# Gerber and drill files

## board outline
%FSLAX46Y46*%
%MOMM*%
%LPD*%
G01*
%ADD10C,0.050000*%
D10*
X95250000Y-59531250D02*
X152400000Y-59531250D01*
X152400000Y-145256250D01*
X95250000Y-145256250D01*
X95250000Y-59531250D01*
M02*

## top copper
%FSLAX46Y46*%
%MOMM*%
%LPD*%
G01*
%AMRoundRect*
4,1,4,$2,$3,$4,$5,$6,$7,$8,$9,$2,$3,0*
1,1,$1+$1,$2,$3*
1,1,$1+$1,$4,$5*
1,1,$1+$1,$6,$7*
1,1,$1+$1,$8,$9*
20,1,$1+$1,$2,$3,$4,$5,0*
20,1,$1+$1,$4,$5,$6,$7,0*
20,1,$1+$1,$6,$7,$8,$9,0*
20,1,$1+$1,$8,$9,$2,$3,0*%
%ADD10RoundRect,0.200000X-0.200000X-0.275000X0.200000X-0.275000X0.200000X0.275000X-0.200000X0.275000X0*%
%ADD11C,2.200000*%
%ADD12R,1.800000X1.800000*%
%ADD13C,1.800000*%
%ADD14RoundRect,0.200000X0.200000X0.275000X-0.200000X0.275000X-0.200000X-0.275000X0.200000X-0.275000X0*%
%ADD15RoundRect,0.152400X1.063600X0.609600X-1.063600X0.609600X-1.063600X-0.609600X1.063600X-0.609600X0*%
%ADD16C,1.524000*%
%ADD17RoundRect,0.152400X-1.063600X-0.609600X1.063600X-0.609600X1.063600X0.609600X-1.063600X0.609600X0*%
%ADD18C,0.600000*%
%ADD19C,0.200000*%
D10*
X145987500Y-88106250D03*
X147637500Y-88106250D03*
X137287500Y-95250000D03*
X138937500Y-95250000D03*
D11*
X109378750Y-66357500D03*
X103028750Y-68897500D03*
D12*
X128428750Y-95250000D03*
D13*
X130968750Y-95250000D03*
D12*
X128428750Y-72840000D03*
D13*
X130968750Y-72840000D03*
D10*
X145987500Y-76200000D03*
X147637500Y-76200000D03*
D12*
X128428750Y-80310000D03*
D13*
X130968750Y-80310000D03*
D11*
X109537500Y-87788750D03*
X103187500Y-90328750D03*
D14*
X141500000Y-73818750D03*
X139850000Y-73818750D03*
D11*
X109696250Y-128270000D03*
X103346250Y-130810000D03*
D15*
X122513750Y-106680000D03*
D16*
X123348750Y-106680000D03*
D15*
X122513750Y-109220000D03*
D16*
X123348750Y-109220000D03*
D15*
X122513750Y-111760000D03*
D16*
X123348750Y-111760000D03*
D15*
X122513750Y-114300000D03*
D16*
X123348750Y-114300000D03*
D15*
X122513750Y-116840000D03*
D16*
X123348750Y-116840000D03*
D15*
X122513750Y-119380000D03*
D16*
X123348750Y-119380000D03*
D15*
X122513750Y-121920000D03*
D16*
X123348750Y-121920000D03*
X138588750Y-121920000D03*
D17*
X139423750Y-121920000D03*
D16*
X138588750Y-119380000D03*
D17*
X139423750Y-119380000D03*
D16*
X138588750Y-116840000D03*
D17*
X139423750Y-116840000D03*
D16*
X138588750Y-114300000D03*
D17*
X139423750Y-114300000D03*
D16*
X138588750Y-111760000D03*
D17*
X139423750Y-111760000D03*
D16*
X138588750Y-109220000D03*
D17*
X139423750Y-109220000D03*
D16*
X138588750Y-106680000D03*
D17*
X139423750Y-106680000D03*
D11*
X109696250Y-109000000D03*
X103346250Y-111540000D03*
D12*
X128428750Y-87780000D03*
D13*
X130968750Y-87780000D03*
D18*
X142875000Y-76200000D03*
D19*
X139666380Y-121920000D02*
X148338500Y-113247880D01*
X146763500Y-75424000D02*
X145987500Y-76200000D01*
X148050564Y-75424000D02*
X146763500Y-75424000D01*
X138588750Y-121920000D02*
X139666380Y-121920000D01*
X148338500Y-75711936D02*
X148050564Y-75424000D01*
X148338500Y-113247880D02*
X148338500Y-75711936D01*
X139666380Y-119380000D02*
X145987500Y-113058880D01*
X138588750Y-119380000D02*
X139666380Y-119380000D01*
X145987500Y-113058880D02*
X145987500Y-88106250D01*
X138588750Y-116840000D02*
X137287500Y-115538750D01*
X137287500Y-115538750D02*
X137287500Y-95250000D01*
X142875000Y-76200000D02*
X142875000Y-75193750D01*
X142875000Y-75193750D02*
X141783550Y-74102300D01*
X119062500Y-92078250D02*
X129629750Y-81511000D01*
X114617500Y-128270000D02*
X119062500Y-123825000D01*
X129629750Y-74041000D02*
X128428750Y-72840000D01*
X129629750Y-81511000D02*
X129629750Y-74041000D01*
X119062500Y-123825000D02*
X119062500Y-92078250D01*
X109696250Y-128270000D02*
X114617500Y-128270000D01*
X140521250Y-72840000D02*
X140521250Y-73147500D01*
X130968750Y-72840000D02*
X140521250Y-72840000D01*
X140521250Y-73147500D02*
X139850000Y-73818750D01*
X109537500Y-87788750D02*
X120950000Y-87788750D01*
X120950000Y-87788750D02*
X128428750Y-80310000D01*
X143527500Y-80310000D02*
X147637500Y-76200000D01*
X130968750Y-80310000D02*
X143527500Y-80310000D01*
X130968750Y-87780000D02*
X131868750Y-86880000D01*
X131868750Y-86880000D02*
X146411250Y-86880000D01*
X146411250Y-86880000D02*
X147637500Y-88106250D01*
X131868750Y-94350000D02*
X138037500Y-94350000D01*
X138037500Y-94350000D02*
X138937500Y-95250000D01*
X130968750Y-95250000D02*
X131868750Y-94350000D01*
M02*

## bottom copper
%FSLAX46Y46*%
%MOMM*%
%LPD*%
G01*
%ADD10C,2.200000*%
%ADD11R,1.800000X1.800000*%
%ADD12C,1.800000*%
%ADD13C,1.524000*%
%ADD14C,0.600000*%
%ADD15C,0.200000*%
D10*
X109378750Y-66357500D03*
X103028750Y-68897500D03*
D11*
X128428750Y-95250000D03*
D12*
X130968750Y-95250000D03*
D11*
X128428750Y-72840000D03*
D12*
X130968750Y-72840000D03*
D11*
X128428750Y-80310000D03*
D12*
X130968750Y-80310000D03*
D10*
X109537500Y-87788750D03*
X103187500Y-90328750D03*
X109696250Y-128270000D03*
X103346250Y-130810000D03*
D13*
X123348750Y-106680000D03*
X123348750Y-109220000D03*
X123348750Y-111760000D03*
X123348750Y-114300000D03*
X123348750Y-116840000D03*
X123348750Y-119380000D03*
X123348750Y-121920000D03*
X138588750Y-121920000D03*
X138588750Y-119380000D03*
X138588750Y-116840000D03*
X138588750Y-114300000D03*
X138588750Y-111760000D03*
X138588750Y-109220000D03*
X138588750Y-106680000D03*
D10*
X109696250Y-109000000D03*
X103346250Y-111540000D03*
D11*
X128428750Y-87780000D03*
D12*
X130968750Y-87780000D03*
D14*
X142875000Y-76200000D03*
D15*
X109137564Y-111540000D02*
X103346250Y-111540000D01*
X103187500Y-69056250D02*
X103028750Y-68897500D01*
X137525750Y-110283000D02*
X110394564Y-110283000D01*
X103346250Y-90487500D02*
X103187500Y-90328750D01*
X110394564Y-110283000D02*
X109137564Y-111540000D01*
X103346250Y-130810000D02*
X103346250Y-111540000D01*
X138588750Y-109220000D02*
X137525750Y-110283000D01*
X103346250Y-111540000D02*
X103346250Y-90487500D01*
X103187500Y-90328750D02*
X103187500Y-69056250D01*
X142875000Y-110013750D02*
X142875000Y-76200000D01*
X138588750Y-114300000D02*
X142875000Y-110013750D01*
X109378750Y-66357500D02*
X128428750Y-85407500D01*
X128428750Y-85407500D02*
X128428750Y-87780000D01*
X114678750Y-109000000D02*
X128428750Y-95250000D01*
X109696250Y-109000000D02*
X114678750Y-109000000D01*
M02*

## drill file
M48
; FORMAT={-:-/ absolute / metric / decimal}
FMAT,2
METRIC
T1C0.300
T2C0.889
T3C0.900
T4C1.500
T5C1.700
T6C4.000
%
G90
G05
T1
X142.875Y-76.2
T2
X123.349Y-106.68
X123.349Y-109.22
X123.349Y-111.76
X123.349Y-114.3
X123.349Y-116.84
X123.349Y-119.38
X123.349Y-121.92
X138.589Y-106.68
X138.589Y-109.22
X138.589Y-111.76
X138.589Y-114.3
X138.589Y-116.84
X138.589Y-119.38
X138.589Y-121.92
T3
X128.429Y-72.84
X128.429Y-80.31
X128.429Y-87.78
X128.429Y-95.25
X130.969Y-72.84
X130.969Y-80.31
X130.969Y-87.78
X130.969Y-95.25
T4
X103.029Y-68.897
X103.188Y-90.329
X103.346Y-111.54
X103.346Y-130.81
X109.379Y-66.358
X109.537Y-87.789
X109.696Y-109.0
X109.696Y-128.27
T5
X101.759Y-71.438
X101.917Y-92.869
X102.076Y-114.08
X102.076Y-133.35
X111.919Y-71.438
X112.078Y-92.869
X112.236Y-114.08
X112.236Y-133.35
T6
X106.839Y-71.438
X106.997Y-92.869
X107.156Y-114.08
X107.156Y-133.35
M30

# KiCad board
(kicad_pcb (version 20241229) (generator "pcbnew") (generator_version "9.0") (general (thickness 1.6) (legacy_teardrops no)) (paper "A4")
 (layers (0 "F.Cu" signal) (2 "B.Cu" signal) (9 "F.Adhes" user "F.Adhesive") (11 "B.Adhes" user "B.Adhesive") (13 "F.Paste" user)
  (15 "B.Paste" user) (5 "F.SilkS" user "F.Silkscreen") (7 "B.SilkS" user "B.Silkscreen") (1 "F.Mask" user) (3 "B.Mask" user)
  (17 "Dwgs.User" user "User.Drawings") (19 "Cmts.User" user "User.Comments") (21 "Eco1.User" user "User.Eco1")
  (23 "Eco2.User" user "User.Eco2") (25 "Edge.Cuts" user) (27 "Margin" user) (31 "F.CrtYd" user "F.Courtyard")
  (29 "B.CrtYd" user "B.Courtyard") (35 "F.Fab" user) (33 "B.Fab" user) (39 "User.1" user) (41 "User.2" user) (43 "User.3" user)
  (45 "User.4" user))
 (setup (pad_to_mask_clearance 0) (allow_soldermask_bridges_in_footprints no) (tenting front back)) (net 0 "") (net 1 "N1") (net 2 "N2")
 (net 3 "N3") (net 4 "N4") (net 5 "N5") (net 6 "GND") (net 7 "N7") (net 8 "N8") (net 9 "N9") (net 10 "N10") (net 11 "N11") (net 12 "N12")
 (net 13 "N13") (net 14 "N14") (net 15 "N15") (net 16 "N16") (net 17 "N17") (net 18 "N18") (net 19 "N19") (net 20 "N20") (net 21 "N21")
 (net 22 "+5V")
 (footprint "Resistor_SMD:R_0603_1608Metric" (layer "F.Cu") (at 146.8125 88.10625)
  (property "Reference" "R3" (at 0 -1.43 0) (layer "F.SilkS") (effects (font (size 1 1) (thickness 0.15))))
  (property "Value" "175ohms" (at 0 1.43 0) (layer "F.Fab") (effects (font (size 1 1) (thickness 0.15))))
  (pad "1" smd roundrect (at -0.825 0) (size 0.8 0.95) (layers "F.Cu" "F.Mask" "F.Paste") (roundrect_rratio 0.25) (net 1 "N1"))
  (pad "2" smd roundrect (at 0.825 0) (size 0.8 0.95) (layers "F.Cu" "F.Mask" "F.Paste") (roundrect_rratio 0.25) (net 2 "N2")))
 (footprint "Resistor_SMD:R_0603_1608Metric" (layer "F.Cu") (at 138.1125 95.25)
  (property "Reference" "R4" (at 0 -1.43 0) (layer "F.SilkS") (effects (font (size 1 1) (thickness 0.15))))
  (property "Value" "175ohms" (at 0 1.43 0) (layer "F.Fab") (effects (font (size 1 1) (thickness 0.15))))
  (pad "1" smd roundrect (at -0.825 0) (size 0.8 0.95) (layers "F.Cu" "F.Mask" "F.Paste") (roundrect_rratio 0.25) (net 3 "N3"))
  (pad "2" smd roundrect (at 0.825 0) (size 0.8 0.95) (layers "F.Cu" "F.Mask" "F.Paste") (roundrect_rratio 0.25) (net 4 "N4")))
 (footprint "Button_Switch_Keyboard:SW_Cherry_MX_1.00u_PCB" (layer "F.Cu") (at 109.37875 66.3575)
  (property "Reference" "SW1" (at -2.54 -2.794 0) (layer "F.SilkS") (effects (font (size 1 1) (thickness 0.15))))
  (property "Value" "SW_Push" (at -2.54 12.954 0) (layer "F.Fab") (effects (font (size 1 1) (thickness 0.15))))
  (pad "" np_thru_hole circle (at -7.62 5.08) (size 1.7 1.7) (drill 1.7) (layers "*.Cu" "*.Mask"))
  (pad "" np_thru_hole circle (at -2.54 5.08) (size 4 4) (drill 4) (layers "*.Cu" "*.Mask"))
  (pad "" np_thru_hole circle (at 2.54 5.08) (size 1.7 1.7) (drill 1.7) (layers "*.Cu" "*.Mask"))
  (pad "1" thru_hole circle (at 0 0) (size 2.2 2.2) (drill 1.5) (layers "*.Cu" "*.Mask") (remove_unused_layers no) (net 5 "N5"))
  (pad "2" thru_hole circle (at -6.35 2.54) (size 2.2 2.2) (drill 1.5) (layers "*.Cu" "*.Mask") (remove_unused_layers no) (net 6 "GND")))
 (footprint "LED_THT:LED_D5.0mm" (layer "F.Cu") (at 128.42875 95.25)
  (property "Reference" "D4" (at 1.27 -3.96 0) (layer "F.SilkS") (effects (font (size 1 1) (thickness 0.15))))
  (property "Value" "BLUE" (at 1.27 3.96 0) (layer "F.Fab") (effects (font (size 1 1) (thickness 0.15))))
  (pad "1" thru_hole rect (at 0 0) (size 1.8 1.8) (drill 0.9) (layers "*.Cu" "*.Mask") (remove_unused_layers no) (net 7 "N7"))
  (pad "2" thru_hole circle (at 2.54 0) (size 1.8 1.8) (drill 0.9) (layers "*.Cu" "*.Mask") (remove_unused_layers no) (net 4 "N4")))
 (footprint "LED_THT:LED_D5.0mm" (layer "F.Cu") (at 128.42875 72.84)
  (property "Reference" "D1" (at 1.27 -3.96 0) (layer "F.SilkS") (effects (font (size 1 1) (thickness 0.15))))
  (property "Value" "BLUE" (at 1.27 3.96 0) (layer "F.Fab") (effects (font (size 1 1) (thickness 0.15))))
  (pad "1" thru_hole rect (at 0 0) (size 1.8 1.8) (drill 0.9) (layers "*.Cu" "*.Mask") (remove_unused_layers no) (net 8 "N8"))
  (pad "2" thru_hole circle (at 2.54 0) (size 1.8 1.8) (drill 0.9) (layers "*.Cu" "*.Mask") (remove_unused_layers no) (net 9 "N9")))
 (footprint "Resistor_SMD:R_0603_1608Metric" (layer "F.Cu") (at 146.8125 76.2)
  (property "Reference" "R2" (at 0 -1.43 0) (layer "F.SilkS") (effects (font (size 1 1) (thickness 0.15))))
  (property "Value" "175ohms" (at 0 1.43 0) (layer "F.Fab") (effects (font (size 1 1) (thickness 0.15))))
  (pad "1" smd roundrect (at -0.825 0) (size 0.8 0.95) (layers "F.Cu" "F.Mask" "F.Paste") (roundrect_rratio 0.25) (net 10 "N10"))
  (pad "2" smd roundrect (at 0.825 0) (size 0.8 0.95) (layers "F.Cu" "F.Mask" "F.Paste") (roundrect_rratio 0.25) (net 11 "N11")))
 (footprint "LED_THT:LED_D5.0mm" (layer "F.Cu") (at 128.42875 80.31)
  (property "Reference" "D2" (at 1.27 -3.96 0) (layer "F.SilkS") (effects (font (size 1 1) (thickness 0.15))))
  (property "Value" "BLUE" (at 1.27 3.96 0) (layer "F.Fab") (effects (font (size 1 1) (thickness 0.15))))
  (pad "1" thru_hole rect (at 0 0) (size 1.8 1.8) (drill 0.9) (layers "*.Cu" "*.Mask") (remove_unused_layers no) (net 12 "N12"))
  (pad "2" thru_hole circle (at 2.54 0) (size 1.8 1.8) (drill 0.9) (layers "*.Cu" "*.Mask") (remove_unused_layers no) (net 11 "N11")))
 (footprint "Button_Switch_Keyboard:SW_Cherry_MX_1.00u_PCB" (layer "F.Cu") (at 109.5375 87.78875)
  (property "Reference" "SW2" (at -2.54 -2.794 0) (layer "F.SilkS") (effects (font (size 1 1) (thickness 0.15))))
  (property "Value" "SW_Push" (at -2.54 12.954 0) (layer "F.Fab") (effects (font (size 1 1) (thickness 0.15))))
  (pad "" np_thru_hole circle (at -7.62 5.08) (size 1.7 1.7) (drill 1.7) (layers "*.Cu" "*.Mask"))
  (pad "" np_thru_hole circle (at -2.54 5.08) (size 4 4) (drill 4) (layers "*.Cu" "*.Mask"))
  (pad "" np_thru_hole circle (at 2.54 5.08) (size 1.7 1.7) (drill 1.7) (layers "*.Cu" "*.Mask"))
  (pad "1" thru_hole circle (at 0 0) (size 2.2 2.2) (drill 1.5) (layers "*.Cu" "*.Mask") (remove_unused_layers no) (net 12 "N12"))
  (pad "2" thru_hole circle (at -6.35 2.54) (size 2.2 2.2) (drill 1.5) (layers "*.Cu" "*.Mask") (remove_unused_layers no) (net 6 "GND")))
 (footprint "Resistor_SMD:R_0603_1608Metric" (layer "F.Cu") (at 140.675 73.81875 180)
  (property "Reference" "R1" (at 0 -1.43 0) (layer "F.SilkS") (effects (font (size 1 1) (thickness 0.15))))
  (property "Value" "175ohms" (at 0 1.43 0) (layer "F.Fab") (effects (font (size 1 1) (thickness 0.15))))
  (pad "1" smd roundrect (at -0.825 0 180) (size 0.8 0.95) (layers "F.Cu" "F.Mask" "F.Paste") (roundrect_rratio 0.25) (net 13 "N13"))
  (pad "2" smd roundrect (at 0.825 0 180) (size 0.8 0.95) (layers "F.Cu" "F.Mask" "F.Paste") (roundrect_rratio 0.25) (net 9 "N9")))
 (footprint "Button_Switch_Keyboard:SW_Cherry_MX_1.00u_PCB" (layer "F.Cu") (at 109.69625 128.27)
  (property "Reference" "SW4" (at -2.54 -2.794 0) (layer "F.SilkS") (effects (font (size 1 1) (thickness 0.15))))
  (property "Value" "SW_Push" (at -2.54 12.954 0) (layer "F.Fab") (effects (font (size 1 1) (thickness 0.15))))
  (pad "" np_thru_hole circle (at -7.62 5.08) (size 1.7 1.7) (drill 1.7) (layers "*.Cu" "*.Mask"))
  (pad "" np_thru_hole circle (at -2.54 5.08) (size 4 4) (drill 4) (layers "*.Cu" "*.Mask"))
  (pad "" np_thru_hole circle (at 2.54 5.08) (size 1.7 1.7) (drill 1.7) (layers "*.Cu" "*.Mask"))
  (pad "1" thru_hole circle (at 0 0) (size 2.2 2.2) (drill 1.5) (layers "*.Cu" "*.Mask") (remove_unused_layers no) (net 8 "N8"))
  (pad "2" thru_hole circle (at -6.35 2.54) (size 2.2 2.2) (drill 1.5) (layers "*.Cu" "*.Mask") (remove_unused_layers no) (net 6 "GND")))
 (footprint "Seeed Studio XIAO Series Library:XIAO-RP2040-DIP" (layer "F.Cu") (at 130.96875 114.3)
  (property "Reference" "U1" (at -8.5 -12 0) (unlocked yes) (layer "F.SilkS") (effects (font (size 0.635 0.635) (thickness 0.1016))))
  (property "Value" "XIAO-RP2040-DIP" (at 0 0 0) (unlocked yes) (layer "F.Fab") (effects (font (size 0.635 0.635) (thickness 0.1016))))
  (pad "1" smd roundrect (at -8.455 -7.62 180) (size 2.432 1.524) (layers "F.Cu" "F.Mask") (roundrect_rratio 0.1) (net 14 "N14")
   (thermal_bridge_angle 45))
  (pad "1" thru_hole circle (at -7.62 -7.62 180) (size 1.524 1.524) (drill 0.889) (layers "*.Cu" "*.Mask") (remove_unused_layers no)
   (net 14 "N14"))
  (pad "2" smd roundrect (at -8.455 -5.08 180) (size 2.432 1.524) (layers "F.Cu" "F.Mask") (roundrect_rratio 0.1) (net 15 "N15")
   (thermal_bridge_angle 45))
  (pad "2" thru_hole circle (at -7.62 -5.08 180) (size 1.524 1.524) (drill 0.889) (layers "*.Cu" "*.Mask") (remove_unused_layers no)
   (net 15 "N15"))
  (pad "3" smd roundrect (at -8.455 -2.54 180) (size 2.432 1.524) (layers "F.Cu" "F.Mask") (roundrect_rratio 0.1) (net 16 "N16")
   (thermal_bridge_angle 45))
  (pad "3" thru_hole circle (at -7.62 -2.54 180) (size 1.524 1.524) (drill 0.889) (layers "*.Cu" "*.Mask") (remove_unused_layers no)
   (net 16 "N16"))
  (pad "4" smd roundrect (at -8.455 0 180) (size 2.432 1.524) (layers "F.Cu" "F.Mask") (roundrect_rratio 0.1) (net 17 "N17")
   (thermal_bridge_angle 45))
  (pad "4" thru_hole circle (at -7.62 0 180) (size 1.524 1.524) (drill 0.889) (layers "*.Cu" "*.Mask") (remove_unused_layers no)
   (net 17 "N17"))
  (pad "5" smd roundrect (at -8.455 2.54 180) (size 2.432 1.524) (layers "F.Cu" "F.Mask") (roundrect_rratio 0.1) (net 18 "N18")
   (thermal_bridge_angle 45))
  (pad "5" thru_hole circle (at -7.62 2.54 180) (size 1.524 1.524) (drill 0.889) (layers "*.Cu" "*.Mask") (remove_unused_layers no)
   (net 18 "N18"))
  (pad "6" smd roundrect (at -8.455 5.08 180) (size 2.432 1.524) (layers "F.Cu" "F.Mask") (roundrect_rratio 0.1) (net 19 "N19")
   (thermal_bridge_angle 45))
  (pad "6" thru_hole circle (at -7.62 5.08 180) (size 1.524 1.524) (drill 0.889) (layers "*.Cu" "*.Mask") (remove_unused_layers no)
   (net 19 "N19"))
  (pad "7" smd roundrect (at -8.455 7.62 180) (size 2.432 1.524) (layers "F.Cu" "F.Mask") (roundrect_rratio 0.1) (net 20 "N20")
   (thermal_bridge_angle 45))
  (pad "7" thru_hole circle (at -7.62 7.62 180) (size 1.524 1.524) (drill 0.889) (layers "*.Cu" "*.Mask") (remove_unused_layers no)
   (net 20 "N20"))
  (pad "8" thru_hole circle (at 7.62 7.62) (size 1.524 1.524) (drill 0.889) (layers "*.Cu" "*.Mask") (remove_unused_layers no)
   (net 10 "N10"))
  (pad "8" smd roundrect (at 8.455 7.62) (size 2.432 1.524) (layers "F.Cu" "F.Mask") (roundrect_rratio 0.1) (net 10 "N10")
   (thermal_bridge_angle 45))
  (pad "9" thru_hole circle (at 7.62 5.08) (size 1.524 1.524) (drill 0.889) (layers "*.Cu" "*.Mask") (remove_unused_layers no) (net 1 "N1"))
  (pad "9" smd roundrect (at 8.455 5.08) (size 2.432 1.524) (layers "F.Cu" "F.Mask") (roundrect_rratio 0.1) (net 1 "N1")
   (thermal_bridge_angle 45))
  (pad "10" thru_hole circle (at 7.62 2.54) (size 1.524 1.524) (drill 0.889) (layers "*.Cu" "*.Mask") (remove_unused_layers no) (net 3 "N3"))
  (pad "10" smd roundrect (at 8.455 2.54) (size 2.432 1.524) (layers "F.Cu" "F.Mask") (roundrect_rratio 0.1) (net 3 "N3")
   (thermal_bridge_angle 45))
  (pad "11" thru_hole circle (at 7.62 0) (size 1.524 1.524) (drill 0.889) (layers "*.Cu" "*.Mask") (remove_unused_layers no) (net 13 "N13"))
  (pad "11" smd roundrect (at 8.455 0) (size 2.432 1.524) (layers "F.Cu" "F.Mask") (roundrect_rratio 0.1) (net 13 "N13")
   (thermal_bridge_angle 45))
  (pad "12" thru_hole circle (at 7.62 -2.54) (size 1.524 1.524) (drill 0.889) (layers "*.Cu" "*.Mask") (remove_unused_layers no)
   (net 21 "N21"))
  (pad "12" smd roundrect (at 8.455 -2.54) (size 2.432 1.524) (layers "F.Cu" "F.Mask") (roundrect_rratio 0.1) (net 21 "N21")
   (thermal_bridge_angle 45))
  (pad "13" thru_hole circle (at 7.62 -5.08) (size 1.524 1.524) (drill 0.889) (layers "*.Cu" "*.Mask") (remove_unused_layers no)
   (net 6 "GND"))
  (pad "13" smd roundrect (at 8.455 -5.08) (size 2.432 1.524) (layers "F.Cu" "F.Mask") (roundrect_rratio 0.1) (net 6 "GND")
   (thermal_bridge_angle 45))
  (pad "14" thru_hole circle (at 7.62 -7.62) (size 1.524 1.524) (drill 0.889) (layers "*.Cu" "*.Mask") (remove_unused_layers no)
   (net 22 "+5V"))
  (pad "14" smd roundrect (at 8.455 -7.62) (size 2.432 1.524) (layers "F.Cu" "F.Mask") (roundrect_rratio 0.1) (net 22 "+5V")
   (thermal_bridge_angle 45)))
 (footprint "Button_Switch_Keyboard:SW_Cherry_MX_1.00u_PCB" (layer "F.Cu") (at 109.69625 109)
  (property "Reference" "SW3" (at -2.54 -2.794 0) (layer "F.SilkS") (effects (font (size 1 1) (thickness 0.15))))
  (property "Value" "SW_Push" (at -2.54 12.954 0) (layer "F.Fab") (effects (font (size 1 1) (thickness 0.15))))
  (pad "" np_thru_hole circle (at -7.62 5.08) (size 1.7 1.7) (drill 1.7) (layers "*.Cu" "*.Mask"))
  (pad "" np_thru_hole circle (at -2.54 5.08) (size 4 4) (drill 4) (layers "*.Cu" "*.Mask"))
  (pad "" np_thru_hole circle (at 2.54 5.08) (size 1.7 1.7) (drill 1.7) (layers "*.Cu" "*.Mask"))
  (pad "1" thru_hole circle (at 0 0) (size 2.2 2.2) (drill 1.5) (layers "*.Cu" "*.Mask") (remove_unused_layers no) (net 7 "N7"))
  (pad "2" thru_hole circle (at -6.35 2.54) (size 2.2 2.2) (drill 1.5) (layers "*.Cu" "*.Mask") (remove_unused_layers no) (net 6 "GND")))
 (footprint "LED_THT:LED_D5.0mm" (layer "F.Cu") (at 128.42875 87.78)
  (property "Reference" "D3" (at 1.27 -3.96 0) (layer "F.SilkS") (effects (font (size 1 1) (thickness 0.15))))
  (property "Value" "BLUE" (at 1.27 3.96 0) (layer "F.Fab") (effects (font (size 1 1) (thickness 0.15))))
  (pad "1" thru_hole rect (at 0 0) (size 1.8 1.8) (drill 0.9) (layers "*.Cu" "*.Mask") (remove_unused_layers no) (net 5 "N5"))
  (pad "2" thru_hole circle (at 2.54 0) (size 1.8 1.8) (drill 0.9) (layers "*.Cu" "*.Mask") (remove_unused_layers no) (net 2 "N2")))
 (gr_rect (start 95.25 59.53125) (end 152.4 145.25625) (stroke (width 0.05) (type default)) (fill no) (layer "Edge.Cuts"))
 (segment (start 109.137564 111.54) (end 103.34625 111.54) (width 0.2) (layer "B.Cu") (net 6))
 (segment (start 103.1875 69.05625) (end 103.02875 68.8975) (width 0.2) (layer "B.Cu") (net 6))
 (segment (start 137.52575 110.283) (end 110.394564 110.283) (width 0.2) (layer "B.Cu") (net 6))
 (segment (start 103.34625 90.4875) (end 103.1875 90.32875) (width 0.2) (layer "B.Cu") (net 6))
 (segment (start 110.394564 110.283) (end 109.137564 111.54) (width 0.2) (layer "B.Cu") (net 6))
 (segment (start 103.34625 130.81) (end 103.34625 111.54) (width 0.2) (layer "B.Cu") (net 6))
 (segment (start 138.58875 109.22) (end 137.52575 110.283) (width 0.2) (layer "B.Cu") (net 6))
 (segment (start 103.34625 111.54) (end 103.34625 90.4875) (width 0.2) (layer "B.Cu") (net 6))
 (segment (start 103.1875 90.32875) (end 103.1875 69.05625) (width 0.2) (layer "B.Cu") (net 6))
 (segment (start 139.66638 121.92) (end 148.3385 113.24788) (width 0.2) (layer "F.Cu") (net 10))
 (segment (start 146.7635 75.424) (end 145.9875 76.2) (width 0.2) (layer "F.Cu") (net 10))
 (segment (start 148.050564 75.424) (end 146.7635 75.424) (width 0.2) (layer "F.Cu") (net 10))
 (segment (start 138.58875 121.92) (end 139.66638 121.92) (width 0.2) (layer "F.Cu") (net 10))
 (segment (start 148.3385 75.711936) (end 148.050564 75.424) (width 0.2) (layer "F.Cu") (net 10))
 (segment (start 148.3385 113.24788) (end 148.3385 75.711936) (width 0.2) (layer "F.Cu") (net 10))
 (segment (start 139.66638 119.38) (end 145.9875 113.05888) (width 0.2) (layer "F.Cu") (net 1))
 (segment (start 138.58875 119.38) (end 139.66638 119.38) (width 0.2) (layer "F.Cu") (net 1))
 (segment (start 145.9875 113.05888) (end 145.9875 88.10625) (width 0.2) (layer "F.Cu") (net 1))
 (segment (start 138.58875 116.84) (end 137.2875 115.53875) (width 0.2) (layer "F.Cu") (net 3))
 (segment (start 137.2875 115.53875) (end 137.2875 95.25) (width 0.2) (layer "F.Cu") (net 3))
 (segment (start 142.875 76.2) (end 142.875 75.19375) (width 0.2) (layer "F.Cu") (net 13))
 (segment (start 142.875 75.19375) (end 141.78355 74.1023) (width 0.2) (layer "F.Cu") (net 13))
 (via (at 142.875 76.2) (size 0.6) (drill 0.3) (layers "F.Cu" "B.Cu") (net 13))
 (segment (start 142.875 110.01375) (end 142.875 76.2) (width 0.2) (layer "B.Cu") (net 13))
 (segment (start 138.58875 114.3) (end 142.875 110.01375) (width 0.2) (layer "B.Cu") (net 13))
 (segment (start 119.0625 92.07825) (end 129.62975 81.511) (width 0.2) (layer "F.Cu") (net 8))
 (segment (start 114.6175 128.27) (end 119.0625 123.825) (width 0.2) (layer "F.Cu") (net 8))
 (segment (start 129.62975 74.041) (end 128.42875 72.84) (width 0.2) (layer "F.Cu") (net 8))
 (segment (start 129.62975 81.511) (end 129.62975 74.041) (width 0.2) (layer "F.Cu") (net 8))
 (segment (start 119.0625 123.825) (end 119.0625 92.07825) (width 0.2) (layer "F.Cu") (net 8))
 (segment (start 109.69625 128.27) (end 114.6175 128.27) (width 0.2) (layer "F.Cu") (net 8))
 (segment (start 140.52125 72.84) (end 140.52125 73.1475) (width 0.2) (layer "F.Cu") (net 9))
 (segment (start 130.96875 72.84) (end 140.52125 72.84) (width 0.2) (layer "F.Cu") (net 9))
 (segment (start 140.52125 73.1475) (end 139.85 73.81875) (width 0.2) (layer "F.Cu") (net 9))
 (segment (start 109.5375 87.78875) (end 120.95 87.78875) (width 0.2) (layer "F.Cu") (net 12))
 (segment (start 120.95 87.78875) (end 128.42875 80.31) (width 0.2) (layer "F.Cu") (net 12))
 (segment (start 143.5275 80.31) (end 147.6375 76.2) (width 0.2) (layer "F.Cu") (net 11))
 (segment (start 130.96875 80.31) (end 143.5275 80.31) (width 0.2) (layer "F.Cu") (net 11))
 (segment (start 109.37875 66.3575) (end 128.42875 85.4075) (width 0.2) (layer "B.Cu") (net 5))
 (segment (start 128.42875 85.4075) (end 128.42875 87.78) (width 0.2) (layer "B.Cu") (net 5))
 (segment (start 130.96875 87.78) (end 131.86875 86.88) (width 0.2) (layer "F.Cu") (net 2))
 (segment (start 131.86875 86.88) (end 146.41125 86.88) (width 0.2) (layer "F.Cu") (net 2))
 (segment (start 146.41125 86.88) (end 147.6375 88.10625) (width 0.2) (layer "F.Cu") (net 2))
 (segment (start 114.67875 109) (end 128.42875 95.25) (width 0.2) (layer "B.Cu") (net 7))
 (segment (start 109.69625 109) (end 114.67875 109) (width 0.2) (layer "B.Cu") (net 7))
 (segment (start 131.86875 94.35) (end 138.0375 94.35) (width 0.2) (layer "F.Cu") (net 4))
 (segment (start 138.0375 94.35) (end 138.9375 95.25) (width 0.2) (layer "F.Cu") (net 4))
 (segment (start 130.96875 95.25) (end 131.86875 94.35) (width 0.2) (layer "F.Cu") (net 4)))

